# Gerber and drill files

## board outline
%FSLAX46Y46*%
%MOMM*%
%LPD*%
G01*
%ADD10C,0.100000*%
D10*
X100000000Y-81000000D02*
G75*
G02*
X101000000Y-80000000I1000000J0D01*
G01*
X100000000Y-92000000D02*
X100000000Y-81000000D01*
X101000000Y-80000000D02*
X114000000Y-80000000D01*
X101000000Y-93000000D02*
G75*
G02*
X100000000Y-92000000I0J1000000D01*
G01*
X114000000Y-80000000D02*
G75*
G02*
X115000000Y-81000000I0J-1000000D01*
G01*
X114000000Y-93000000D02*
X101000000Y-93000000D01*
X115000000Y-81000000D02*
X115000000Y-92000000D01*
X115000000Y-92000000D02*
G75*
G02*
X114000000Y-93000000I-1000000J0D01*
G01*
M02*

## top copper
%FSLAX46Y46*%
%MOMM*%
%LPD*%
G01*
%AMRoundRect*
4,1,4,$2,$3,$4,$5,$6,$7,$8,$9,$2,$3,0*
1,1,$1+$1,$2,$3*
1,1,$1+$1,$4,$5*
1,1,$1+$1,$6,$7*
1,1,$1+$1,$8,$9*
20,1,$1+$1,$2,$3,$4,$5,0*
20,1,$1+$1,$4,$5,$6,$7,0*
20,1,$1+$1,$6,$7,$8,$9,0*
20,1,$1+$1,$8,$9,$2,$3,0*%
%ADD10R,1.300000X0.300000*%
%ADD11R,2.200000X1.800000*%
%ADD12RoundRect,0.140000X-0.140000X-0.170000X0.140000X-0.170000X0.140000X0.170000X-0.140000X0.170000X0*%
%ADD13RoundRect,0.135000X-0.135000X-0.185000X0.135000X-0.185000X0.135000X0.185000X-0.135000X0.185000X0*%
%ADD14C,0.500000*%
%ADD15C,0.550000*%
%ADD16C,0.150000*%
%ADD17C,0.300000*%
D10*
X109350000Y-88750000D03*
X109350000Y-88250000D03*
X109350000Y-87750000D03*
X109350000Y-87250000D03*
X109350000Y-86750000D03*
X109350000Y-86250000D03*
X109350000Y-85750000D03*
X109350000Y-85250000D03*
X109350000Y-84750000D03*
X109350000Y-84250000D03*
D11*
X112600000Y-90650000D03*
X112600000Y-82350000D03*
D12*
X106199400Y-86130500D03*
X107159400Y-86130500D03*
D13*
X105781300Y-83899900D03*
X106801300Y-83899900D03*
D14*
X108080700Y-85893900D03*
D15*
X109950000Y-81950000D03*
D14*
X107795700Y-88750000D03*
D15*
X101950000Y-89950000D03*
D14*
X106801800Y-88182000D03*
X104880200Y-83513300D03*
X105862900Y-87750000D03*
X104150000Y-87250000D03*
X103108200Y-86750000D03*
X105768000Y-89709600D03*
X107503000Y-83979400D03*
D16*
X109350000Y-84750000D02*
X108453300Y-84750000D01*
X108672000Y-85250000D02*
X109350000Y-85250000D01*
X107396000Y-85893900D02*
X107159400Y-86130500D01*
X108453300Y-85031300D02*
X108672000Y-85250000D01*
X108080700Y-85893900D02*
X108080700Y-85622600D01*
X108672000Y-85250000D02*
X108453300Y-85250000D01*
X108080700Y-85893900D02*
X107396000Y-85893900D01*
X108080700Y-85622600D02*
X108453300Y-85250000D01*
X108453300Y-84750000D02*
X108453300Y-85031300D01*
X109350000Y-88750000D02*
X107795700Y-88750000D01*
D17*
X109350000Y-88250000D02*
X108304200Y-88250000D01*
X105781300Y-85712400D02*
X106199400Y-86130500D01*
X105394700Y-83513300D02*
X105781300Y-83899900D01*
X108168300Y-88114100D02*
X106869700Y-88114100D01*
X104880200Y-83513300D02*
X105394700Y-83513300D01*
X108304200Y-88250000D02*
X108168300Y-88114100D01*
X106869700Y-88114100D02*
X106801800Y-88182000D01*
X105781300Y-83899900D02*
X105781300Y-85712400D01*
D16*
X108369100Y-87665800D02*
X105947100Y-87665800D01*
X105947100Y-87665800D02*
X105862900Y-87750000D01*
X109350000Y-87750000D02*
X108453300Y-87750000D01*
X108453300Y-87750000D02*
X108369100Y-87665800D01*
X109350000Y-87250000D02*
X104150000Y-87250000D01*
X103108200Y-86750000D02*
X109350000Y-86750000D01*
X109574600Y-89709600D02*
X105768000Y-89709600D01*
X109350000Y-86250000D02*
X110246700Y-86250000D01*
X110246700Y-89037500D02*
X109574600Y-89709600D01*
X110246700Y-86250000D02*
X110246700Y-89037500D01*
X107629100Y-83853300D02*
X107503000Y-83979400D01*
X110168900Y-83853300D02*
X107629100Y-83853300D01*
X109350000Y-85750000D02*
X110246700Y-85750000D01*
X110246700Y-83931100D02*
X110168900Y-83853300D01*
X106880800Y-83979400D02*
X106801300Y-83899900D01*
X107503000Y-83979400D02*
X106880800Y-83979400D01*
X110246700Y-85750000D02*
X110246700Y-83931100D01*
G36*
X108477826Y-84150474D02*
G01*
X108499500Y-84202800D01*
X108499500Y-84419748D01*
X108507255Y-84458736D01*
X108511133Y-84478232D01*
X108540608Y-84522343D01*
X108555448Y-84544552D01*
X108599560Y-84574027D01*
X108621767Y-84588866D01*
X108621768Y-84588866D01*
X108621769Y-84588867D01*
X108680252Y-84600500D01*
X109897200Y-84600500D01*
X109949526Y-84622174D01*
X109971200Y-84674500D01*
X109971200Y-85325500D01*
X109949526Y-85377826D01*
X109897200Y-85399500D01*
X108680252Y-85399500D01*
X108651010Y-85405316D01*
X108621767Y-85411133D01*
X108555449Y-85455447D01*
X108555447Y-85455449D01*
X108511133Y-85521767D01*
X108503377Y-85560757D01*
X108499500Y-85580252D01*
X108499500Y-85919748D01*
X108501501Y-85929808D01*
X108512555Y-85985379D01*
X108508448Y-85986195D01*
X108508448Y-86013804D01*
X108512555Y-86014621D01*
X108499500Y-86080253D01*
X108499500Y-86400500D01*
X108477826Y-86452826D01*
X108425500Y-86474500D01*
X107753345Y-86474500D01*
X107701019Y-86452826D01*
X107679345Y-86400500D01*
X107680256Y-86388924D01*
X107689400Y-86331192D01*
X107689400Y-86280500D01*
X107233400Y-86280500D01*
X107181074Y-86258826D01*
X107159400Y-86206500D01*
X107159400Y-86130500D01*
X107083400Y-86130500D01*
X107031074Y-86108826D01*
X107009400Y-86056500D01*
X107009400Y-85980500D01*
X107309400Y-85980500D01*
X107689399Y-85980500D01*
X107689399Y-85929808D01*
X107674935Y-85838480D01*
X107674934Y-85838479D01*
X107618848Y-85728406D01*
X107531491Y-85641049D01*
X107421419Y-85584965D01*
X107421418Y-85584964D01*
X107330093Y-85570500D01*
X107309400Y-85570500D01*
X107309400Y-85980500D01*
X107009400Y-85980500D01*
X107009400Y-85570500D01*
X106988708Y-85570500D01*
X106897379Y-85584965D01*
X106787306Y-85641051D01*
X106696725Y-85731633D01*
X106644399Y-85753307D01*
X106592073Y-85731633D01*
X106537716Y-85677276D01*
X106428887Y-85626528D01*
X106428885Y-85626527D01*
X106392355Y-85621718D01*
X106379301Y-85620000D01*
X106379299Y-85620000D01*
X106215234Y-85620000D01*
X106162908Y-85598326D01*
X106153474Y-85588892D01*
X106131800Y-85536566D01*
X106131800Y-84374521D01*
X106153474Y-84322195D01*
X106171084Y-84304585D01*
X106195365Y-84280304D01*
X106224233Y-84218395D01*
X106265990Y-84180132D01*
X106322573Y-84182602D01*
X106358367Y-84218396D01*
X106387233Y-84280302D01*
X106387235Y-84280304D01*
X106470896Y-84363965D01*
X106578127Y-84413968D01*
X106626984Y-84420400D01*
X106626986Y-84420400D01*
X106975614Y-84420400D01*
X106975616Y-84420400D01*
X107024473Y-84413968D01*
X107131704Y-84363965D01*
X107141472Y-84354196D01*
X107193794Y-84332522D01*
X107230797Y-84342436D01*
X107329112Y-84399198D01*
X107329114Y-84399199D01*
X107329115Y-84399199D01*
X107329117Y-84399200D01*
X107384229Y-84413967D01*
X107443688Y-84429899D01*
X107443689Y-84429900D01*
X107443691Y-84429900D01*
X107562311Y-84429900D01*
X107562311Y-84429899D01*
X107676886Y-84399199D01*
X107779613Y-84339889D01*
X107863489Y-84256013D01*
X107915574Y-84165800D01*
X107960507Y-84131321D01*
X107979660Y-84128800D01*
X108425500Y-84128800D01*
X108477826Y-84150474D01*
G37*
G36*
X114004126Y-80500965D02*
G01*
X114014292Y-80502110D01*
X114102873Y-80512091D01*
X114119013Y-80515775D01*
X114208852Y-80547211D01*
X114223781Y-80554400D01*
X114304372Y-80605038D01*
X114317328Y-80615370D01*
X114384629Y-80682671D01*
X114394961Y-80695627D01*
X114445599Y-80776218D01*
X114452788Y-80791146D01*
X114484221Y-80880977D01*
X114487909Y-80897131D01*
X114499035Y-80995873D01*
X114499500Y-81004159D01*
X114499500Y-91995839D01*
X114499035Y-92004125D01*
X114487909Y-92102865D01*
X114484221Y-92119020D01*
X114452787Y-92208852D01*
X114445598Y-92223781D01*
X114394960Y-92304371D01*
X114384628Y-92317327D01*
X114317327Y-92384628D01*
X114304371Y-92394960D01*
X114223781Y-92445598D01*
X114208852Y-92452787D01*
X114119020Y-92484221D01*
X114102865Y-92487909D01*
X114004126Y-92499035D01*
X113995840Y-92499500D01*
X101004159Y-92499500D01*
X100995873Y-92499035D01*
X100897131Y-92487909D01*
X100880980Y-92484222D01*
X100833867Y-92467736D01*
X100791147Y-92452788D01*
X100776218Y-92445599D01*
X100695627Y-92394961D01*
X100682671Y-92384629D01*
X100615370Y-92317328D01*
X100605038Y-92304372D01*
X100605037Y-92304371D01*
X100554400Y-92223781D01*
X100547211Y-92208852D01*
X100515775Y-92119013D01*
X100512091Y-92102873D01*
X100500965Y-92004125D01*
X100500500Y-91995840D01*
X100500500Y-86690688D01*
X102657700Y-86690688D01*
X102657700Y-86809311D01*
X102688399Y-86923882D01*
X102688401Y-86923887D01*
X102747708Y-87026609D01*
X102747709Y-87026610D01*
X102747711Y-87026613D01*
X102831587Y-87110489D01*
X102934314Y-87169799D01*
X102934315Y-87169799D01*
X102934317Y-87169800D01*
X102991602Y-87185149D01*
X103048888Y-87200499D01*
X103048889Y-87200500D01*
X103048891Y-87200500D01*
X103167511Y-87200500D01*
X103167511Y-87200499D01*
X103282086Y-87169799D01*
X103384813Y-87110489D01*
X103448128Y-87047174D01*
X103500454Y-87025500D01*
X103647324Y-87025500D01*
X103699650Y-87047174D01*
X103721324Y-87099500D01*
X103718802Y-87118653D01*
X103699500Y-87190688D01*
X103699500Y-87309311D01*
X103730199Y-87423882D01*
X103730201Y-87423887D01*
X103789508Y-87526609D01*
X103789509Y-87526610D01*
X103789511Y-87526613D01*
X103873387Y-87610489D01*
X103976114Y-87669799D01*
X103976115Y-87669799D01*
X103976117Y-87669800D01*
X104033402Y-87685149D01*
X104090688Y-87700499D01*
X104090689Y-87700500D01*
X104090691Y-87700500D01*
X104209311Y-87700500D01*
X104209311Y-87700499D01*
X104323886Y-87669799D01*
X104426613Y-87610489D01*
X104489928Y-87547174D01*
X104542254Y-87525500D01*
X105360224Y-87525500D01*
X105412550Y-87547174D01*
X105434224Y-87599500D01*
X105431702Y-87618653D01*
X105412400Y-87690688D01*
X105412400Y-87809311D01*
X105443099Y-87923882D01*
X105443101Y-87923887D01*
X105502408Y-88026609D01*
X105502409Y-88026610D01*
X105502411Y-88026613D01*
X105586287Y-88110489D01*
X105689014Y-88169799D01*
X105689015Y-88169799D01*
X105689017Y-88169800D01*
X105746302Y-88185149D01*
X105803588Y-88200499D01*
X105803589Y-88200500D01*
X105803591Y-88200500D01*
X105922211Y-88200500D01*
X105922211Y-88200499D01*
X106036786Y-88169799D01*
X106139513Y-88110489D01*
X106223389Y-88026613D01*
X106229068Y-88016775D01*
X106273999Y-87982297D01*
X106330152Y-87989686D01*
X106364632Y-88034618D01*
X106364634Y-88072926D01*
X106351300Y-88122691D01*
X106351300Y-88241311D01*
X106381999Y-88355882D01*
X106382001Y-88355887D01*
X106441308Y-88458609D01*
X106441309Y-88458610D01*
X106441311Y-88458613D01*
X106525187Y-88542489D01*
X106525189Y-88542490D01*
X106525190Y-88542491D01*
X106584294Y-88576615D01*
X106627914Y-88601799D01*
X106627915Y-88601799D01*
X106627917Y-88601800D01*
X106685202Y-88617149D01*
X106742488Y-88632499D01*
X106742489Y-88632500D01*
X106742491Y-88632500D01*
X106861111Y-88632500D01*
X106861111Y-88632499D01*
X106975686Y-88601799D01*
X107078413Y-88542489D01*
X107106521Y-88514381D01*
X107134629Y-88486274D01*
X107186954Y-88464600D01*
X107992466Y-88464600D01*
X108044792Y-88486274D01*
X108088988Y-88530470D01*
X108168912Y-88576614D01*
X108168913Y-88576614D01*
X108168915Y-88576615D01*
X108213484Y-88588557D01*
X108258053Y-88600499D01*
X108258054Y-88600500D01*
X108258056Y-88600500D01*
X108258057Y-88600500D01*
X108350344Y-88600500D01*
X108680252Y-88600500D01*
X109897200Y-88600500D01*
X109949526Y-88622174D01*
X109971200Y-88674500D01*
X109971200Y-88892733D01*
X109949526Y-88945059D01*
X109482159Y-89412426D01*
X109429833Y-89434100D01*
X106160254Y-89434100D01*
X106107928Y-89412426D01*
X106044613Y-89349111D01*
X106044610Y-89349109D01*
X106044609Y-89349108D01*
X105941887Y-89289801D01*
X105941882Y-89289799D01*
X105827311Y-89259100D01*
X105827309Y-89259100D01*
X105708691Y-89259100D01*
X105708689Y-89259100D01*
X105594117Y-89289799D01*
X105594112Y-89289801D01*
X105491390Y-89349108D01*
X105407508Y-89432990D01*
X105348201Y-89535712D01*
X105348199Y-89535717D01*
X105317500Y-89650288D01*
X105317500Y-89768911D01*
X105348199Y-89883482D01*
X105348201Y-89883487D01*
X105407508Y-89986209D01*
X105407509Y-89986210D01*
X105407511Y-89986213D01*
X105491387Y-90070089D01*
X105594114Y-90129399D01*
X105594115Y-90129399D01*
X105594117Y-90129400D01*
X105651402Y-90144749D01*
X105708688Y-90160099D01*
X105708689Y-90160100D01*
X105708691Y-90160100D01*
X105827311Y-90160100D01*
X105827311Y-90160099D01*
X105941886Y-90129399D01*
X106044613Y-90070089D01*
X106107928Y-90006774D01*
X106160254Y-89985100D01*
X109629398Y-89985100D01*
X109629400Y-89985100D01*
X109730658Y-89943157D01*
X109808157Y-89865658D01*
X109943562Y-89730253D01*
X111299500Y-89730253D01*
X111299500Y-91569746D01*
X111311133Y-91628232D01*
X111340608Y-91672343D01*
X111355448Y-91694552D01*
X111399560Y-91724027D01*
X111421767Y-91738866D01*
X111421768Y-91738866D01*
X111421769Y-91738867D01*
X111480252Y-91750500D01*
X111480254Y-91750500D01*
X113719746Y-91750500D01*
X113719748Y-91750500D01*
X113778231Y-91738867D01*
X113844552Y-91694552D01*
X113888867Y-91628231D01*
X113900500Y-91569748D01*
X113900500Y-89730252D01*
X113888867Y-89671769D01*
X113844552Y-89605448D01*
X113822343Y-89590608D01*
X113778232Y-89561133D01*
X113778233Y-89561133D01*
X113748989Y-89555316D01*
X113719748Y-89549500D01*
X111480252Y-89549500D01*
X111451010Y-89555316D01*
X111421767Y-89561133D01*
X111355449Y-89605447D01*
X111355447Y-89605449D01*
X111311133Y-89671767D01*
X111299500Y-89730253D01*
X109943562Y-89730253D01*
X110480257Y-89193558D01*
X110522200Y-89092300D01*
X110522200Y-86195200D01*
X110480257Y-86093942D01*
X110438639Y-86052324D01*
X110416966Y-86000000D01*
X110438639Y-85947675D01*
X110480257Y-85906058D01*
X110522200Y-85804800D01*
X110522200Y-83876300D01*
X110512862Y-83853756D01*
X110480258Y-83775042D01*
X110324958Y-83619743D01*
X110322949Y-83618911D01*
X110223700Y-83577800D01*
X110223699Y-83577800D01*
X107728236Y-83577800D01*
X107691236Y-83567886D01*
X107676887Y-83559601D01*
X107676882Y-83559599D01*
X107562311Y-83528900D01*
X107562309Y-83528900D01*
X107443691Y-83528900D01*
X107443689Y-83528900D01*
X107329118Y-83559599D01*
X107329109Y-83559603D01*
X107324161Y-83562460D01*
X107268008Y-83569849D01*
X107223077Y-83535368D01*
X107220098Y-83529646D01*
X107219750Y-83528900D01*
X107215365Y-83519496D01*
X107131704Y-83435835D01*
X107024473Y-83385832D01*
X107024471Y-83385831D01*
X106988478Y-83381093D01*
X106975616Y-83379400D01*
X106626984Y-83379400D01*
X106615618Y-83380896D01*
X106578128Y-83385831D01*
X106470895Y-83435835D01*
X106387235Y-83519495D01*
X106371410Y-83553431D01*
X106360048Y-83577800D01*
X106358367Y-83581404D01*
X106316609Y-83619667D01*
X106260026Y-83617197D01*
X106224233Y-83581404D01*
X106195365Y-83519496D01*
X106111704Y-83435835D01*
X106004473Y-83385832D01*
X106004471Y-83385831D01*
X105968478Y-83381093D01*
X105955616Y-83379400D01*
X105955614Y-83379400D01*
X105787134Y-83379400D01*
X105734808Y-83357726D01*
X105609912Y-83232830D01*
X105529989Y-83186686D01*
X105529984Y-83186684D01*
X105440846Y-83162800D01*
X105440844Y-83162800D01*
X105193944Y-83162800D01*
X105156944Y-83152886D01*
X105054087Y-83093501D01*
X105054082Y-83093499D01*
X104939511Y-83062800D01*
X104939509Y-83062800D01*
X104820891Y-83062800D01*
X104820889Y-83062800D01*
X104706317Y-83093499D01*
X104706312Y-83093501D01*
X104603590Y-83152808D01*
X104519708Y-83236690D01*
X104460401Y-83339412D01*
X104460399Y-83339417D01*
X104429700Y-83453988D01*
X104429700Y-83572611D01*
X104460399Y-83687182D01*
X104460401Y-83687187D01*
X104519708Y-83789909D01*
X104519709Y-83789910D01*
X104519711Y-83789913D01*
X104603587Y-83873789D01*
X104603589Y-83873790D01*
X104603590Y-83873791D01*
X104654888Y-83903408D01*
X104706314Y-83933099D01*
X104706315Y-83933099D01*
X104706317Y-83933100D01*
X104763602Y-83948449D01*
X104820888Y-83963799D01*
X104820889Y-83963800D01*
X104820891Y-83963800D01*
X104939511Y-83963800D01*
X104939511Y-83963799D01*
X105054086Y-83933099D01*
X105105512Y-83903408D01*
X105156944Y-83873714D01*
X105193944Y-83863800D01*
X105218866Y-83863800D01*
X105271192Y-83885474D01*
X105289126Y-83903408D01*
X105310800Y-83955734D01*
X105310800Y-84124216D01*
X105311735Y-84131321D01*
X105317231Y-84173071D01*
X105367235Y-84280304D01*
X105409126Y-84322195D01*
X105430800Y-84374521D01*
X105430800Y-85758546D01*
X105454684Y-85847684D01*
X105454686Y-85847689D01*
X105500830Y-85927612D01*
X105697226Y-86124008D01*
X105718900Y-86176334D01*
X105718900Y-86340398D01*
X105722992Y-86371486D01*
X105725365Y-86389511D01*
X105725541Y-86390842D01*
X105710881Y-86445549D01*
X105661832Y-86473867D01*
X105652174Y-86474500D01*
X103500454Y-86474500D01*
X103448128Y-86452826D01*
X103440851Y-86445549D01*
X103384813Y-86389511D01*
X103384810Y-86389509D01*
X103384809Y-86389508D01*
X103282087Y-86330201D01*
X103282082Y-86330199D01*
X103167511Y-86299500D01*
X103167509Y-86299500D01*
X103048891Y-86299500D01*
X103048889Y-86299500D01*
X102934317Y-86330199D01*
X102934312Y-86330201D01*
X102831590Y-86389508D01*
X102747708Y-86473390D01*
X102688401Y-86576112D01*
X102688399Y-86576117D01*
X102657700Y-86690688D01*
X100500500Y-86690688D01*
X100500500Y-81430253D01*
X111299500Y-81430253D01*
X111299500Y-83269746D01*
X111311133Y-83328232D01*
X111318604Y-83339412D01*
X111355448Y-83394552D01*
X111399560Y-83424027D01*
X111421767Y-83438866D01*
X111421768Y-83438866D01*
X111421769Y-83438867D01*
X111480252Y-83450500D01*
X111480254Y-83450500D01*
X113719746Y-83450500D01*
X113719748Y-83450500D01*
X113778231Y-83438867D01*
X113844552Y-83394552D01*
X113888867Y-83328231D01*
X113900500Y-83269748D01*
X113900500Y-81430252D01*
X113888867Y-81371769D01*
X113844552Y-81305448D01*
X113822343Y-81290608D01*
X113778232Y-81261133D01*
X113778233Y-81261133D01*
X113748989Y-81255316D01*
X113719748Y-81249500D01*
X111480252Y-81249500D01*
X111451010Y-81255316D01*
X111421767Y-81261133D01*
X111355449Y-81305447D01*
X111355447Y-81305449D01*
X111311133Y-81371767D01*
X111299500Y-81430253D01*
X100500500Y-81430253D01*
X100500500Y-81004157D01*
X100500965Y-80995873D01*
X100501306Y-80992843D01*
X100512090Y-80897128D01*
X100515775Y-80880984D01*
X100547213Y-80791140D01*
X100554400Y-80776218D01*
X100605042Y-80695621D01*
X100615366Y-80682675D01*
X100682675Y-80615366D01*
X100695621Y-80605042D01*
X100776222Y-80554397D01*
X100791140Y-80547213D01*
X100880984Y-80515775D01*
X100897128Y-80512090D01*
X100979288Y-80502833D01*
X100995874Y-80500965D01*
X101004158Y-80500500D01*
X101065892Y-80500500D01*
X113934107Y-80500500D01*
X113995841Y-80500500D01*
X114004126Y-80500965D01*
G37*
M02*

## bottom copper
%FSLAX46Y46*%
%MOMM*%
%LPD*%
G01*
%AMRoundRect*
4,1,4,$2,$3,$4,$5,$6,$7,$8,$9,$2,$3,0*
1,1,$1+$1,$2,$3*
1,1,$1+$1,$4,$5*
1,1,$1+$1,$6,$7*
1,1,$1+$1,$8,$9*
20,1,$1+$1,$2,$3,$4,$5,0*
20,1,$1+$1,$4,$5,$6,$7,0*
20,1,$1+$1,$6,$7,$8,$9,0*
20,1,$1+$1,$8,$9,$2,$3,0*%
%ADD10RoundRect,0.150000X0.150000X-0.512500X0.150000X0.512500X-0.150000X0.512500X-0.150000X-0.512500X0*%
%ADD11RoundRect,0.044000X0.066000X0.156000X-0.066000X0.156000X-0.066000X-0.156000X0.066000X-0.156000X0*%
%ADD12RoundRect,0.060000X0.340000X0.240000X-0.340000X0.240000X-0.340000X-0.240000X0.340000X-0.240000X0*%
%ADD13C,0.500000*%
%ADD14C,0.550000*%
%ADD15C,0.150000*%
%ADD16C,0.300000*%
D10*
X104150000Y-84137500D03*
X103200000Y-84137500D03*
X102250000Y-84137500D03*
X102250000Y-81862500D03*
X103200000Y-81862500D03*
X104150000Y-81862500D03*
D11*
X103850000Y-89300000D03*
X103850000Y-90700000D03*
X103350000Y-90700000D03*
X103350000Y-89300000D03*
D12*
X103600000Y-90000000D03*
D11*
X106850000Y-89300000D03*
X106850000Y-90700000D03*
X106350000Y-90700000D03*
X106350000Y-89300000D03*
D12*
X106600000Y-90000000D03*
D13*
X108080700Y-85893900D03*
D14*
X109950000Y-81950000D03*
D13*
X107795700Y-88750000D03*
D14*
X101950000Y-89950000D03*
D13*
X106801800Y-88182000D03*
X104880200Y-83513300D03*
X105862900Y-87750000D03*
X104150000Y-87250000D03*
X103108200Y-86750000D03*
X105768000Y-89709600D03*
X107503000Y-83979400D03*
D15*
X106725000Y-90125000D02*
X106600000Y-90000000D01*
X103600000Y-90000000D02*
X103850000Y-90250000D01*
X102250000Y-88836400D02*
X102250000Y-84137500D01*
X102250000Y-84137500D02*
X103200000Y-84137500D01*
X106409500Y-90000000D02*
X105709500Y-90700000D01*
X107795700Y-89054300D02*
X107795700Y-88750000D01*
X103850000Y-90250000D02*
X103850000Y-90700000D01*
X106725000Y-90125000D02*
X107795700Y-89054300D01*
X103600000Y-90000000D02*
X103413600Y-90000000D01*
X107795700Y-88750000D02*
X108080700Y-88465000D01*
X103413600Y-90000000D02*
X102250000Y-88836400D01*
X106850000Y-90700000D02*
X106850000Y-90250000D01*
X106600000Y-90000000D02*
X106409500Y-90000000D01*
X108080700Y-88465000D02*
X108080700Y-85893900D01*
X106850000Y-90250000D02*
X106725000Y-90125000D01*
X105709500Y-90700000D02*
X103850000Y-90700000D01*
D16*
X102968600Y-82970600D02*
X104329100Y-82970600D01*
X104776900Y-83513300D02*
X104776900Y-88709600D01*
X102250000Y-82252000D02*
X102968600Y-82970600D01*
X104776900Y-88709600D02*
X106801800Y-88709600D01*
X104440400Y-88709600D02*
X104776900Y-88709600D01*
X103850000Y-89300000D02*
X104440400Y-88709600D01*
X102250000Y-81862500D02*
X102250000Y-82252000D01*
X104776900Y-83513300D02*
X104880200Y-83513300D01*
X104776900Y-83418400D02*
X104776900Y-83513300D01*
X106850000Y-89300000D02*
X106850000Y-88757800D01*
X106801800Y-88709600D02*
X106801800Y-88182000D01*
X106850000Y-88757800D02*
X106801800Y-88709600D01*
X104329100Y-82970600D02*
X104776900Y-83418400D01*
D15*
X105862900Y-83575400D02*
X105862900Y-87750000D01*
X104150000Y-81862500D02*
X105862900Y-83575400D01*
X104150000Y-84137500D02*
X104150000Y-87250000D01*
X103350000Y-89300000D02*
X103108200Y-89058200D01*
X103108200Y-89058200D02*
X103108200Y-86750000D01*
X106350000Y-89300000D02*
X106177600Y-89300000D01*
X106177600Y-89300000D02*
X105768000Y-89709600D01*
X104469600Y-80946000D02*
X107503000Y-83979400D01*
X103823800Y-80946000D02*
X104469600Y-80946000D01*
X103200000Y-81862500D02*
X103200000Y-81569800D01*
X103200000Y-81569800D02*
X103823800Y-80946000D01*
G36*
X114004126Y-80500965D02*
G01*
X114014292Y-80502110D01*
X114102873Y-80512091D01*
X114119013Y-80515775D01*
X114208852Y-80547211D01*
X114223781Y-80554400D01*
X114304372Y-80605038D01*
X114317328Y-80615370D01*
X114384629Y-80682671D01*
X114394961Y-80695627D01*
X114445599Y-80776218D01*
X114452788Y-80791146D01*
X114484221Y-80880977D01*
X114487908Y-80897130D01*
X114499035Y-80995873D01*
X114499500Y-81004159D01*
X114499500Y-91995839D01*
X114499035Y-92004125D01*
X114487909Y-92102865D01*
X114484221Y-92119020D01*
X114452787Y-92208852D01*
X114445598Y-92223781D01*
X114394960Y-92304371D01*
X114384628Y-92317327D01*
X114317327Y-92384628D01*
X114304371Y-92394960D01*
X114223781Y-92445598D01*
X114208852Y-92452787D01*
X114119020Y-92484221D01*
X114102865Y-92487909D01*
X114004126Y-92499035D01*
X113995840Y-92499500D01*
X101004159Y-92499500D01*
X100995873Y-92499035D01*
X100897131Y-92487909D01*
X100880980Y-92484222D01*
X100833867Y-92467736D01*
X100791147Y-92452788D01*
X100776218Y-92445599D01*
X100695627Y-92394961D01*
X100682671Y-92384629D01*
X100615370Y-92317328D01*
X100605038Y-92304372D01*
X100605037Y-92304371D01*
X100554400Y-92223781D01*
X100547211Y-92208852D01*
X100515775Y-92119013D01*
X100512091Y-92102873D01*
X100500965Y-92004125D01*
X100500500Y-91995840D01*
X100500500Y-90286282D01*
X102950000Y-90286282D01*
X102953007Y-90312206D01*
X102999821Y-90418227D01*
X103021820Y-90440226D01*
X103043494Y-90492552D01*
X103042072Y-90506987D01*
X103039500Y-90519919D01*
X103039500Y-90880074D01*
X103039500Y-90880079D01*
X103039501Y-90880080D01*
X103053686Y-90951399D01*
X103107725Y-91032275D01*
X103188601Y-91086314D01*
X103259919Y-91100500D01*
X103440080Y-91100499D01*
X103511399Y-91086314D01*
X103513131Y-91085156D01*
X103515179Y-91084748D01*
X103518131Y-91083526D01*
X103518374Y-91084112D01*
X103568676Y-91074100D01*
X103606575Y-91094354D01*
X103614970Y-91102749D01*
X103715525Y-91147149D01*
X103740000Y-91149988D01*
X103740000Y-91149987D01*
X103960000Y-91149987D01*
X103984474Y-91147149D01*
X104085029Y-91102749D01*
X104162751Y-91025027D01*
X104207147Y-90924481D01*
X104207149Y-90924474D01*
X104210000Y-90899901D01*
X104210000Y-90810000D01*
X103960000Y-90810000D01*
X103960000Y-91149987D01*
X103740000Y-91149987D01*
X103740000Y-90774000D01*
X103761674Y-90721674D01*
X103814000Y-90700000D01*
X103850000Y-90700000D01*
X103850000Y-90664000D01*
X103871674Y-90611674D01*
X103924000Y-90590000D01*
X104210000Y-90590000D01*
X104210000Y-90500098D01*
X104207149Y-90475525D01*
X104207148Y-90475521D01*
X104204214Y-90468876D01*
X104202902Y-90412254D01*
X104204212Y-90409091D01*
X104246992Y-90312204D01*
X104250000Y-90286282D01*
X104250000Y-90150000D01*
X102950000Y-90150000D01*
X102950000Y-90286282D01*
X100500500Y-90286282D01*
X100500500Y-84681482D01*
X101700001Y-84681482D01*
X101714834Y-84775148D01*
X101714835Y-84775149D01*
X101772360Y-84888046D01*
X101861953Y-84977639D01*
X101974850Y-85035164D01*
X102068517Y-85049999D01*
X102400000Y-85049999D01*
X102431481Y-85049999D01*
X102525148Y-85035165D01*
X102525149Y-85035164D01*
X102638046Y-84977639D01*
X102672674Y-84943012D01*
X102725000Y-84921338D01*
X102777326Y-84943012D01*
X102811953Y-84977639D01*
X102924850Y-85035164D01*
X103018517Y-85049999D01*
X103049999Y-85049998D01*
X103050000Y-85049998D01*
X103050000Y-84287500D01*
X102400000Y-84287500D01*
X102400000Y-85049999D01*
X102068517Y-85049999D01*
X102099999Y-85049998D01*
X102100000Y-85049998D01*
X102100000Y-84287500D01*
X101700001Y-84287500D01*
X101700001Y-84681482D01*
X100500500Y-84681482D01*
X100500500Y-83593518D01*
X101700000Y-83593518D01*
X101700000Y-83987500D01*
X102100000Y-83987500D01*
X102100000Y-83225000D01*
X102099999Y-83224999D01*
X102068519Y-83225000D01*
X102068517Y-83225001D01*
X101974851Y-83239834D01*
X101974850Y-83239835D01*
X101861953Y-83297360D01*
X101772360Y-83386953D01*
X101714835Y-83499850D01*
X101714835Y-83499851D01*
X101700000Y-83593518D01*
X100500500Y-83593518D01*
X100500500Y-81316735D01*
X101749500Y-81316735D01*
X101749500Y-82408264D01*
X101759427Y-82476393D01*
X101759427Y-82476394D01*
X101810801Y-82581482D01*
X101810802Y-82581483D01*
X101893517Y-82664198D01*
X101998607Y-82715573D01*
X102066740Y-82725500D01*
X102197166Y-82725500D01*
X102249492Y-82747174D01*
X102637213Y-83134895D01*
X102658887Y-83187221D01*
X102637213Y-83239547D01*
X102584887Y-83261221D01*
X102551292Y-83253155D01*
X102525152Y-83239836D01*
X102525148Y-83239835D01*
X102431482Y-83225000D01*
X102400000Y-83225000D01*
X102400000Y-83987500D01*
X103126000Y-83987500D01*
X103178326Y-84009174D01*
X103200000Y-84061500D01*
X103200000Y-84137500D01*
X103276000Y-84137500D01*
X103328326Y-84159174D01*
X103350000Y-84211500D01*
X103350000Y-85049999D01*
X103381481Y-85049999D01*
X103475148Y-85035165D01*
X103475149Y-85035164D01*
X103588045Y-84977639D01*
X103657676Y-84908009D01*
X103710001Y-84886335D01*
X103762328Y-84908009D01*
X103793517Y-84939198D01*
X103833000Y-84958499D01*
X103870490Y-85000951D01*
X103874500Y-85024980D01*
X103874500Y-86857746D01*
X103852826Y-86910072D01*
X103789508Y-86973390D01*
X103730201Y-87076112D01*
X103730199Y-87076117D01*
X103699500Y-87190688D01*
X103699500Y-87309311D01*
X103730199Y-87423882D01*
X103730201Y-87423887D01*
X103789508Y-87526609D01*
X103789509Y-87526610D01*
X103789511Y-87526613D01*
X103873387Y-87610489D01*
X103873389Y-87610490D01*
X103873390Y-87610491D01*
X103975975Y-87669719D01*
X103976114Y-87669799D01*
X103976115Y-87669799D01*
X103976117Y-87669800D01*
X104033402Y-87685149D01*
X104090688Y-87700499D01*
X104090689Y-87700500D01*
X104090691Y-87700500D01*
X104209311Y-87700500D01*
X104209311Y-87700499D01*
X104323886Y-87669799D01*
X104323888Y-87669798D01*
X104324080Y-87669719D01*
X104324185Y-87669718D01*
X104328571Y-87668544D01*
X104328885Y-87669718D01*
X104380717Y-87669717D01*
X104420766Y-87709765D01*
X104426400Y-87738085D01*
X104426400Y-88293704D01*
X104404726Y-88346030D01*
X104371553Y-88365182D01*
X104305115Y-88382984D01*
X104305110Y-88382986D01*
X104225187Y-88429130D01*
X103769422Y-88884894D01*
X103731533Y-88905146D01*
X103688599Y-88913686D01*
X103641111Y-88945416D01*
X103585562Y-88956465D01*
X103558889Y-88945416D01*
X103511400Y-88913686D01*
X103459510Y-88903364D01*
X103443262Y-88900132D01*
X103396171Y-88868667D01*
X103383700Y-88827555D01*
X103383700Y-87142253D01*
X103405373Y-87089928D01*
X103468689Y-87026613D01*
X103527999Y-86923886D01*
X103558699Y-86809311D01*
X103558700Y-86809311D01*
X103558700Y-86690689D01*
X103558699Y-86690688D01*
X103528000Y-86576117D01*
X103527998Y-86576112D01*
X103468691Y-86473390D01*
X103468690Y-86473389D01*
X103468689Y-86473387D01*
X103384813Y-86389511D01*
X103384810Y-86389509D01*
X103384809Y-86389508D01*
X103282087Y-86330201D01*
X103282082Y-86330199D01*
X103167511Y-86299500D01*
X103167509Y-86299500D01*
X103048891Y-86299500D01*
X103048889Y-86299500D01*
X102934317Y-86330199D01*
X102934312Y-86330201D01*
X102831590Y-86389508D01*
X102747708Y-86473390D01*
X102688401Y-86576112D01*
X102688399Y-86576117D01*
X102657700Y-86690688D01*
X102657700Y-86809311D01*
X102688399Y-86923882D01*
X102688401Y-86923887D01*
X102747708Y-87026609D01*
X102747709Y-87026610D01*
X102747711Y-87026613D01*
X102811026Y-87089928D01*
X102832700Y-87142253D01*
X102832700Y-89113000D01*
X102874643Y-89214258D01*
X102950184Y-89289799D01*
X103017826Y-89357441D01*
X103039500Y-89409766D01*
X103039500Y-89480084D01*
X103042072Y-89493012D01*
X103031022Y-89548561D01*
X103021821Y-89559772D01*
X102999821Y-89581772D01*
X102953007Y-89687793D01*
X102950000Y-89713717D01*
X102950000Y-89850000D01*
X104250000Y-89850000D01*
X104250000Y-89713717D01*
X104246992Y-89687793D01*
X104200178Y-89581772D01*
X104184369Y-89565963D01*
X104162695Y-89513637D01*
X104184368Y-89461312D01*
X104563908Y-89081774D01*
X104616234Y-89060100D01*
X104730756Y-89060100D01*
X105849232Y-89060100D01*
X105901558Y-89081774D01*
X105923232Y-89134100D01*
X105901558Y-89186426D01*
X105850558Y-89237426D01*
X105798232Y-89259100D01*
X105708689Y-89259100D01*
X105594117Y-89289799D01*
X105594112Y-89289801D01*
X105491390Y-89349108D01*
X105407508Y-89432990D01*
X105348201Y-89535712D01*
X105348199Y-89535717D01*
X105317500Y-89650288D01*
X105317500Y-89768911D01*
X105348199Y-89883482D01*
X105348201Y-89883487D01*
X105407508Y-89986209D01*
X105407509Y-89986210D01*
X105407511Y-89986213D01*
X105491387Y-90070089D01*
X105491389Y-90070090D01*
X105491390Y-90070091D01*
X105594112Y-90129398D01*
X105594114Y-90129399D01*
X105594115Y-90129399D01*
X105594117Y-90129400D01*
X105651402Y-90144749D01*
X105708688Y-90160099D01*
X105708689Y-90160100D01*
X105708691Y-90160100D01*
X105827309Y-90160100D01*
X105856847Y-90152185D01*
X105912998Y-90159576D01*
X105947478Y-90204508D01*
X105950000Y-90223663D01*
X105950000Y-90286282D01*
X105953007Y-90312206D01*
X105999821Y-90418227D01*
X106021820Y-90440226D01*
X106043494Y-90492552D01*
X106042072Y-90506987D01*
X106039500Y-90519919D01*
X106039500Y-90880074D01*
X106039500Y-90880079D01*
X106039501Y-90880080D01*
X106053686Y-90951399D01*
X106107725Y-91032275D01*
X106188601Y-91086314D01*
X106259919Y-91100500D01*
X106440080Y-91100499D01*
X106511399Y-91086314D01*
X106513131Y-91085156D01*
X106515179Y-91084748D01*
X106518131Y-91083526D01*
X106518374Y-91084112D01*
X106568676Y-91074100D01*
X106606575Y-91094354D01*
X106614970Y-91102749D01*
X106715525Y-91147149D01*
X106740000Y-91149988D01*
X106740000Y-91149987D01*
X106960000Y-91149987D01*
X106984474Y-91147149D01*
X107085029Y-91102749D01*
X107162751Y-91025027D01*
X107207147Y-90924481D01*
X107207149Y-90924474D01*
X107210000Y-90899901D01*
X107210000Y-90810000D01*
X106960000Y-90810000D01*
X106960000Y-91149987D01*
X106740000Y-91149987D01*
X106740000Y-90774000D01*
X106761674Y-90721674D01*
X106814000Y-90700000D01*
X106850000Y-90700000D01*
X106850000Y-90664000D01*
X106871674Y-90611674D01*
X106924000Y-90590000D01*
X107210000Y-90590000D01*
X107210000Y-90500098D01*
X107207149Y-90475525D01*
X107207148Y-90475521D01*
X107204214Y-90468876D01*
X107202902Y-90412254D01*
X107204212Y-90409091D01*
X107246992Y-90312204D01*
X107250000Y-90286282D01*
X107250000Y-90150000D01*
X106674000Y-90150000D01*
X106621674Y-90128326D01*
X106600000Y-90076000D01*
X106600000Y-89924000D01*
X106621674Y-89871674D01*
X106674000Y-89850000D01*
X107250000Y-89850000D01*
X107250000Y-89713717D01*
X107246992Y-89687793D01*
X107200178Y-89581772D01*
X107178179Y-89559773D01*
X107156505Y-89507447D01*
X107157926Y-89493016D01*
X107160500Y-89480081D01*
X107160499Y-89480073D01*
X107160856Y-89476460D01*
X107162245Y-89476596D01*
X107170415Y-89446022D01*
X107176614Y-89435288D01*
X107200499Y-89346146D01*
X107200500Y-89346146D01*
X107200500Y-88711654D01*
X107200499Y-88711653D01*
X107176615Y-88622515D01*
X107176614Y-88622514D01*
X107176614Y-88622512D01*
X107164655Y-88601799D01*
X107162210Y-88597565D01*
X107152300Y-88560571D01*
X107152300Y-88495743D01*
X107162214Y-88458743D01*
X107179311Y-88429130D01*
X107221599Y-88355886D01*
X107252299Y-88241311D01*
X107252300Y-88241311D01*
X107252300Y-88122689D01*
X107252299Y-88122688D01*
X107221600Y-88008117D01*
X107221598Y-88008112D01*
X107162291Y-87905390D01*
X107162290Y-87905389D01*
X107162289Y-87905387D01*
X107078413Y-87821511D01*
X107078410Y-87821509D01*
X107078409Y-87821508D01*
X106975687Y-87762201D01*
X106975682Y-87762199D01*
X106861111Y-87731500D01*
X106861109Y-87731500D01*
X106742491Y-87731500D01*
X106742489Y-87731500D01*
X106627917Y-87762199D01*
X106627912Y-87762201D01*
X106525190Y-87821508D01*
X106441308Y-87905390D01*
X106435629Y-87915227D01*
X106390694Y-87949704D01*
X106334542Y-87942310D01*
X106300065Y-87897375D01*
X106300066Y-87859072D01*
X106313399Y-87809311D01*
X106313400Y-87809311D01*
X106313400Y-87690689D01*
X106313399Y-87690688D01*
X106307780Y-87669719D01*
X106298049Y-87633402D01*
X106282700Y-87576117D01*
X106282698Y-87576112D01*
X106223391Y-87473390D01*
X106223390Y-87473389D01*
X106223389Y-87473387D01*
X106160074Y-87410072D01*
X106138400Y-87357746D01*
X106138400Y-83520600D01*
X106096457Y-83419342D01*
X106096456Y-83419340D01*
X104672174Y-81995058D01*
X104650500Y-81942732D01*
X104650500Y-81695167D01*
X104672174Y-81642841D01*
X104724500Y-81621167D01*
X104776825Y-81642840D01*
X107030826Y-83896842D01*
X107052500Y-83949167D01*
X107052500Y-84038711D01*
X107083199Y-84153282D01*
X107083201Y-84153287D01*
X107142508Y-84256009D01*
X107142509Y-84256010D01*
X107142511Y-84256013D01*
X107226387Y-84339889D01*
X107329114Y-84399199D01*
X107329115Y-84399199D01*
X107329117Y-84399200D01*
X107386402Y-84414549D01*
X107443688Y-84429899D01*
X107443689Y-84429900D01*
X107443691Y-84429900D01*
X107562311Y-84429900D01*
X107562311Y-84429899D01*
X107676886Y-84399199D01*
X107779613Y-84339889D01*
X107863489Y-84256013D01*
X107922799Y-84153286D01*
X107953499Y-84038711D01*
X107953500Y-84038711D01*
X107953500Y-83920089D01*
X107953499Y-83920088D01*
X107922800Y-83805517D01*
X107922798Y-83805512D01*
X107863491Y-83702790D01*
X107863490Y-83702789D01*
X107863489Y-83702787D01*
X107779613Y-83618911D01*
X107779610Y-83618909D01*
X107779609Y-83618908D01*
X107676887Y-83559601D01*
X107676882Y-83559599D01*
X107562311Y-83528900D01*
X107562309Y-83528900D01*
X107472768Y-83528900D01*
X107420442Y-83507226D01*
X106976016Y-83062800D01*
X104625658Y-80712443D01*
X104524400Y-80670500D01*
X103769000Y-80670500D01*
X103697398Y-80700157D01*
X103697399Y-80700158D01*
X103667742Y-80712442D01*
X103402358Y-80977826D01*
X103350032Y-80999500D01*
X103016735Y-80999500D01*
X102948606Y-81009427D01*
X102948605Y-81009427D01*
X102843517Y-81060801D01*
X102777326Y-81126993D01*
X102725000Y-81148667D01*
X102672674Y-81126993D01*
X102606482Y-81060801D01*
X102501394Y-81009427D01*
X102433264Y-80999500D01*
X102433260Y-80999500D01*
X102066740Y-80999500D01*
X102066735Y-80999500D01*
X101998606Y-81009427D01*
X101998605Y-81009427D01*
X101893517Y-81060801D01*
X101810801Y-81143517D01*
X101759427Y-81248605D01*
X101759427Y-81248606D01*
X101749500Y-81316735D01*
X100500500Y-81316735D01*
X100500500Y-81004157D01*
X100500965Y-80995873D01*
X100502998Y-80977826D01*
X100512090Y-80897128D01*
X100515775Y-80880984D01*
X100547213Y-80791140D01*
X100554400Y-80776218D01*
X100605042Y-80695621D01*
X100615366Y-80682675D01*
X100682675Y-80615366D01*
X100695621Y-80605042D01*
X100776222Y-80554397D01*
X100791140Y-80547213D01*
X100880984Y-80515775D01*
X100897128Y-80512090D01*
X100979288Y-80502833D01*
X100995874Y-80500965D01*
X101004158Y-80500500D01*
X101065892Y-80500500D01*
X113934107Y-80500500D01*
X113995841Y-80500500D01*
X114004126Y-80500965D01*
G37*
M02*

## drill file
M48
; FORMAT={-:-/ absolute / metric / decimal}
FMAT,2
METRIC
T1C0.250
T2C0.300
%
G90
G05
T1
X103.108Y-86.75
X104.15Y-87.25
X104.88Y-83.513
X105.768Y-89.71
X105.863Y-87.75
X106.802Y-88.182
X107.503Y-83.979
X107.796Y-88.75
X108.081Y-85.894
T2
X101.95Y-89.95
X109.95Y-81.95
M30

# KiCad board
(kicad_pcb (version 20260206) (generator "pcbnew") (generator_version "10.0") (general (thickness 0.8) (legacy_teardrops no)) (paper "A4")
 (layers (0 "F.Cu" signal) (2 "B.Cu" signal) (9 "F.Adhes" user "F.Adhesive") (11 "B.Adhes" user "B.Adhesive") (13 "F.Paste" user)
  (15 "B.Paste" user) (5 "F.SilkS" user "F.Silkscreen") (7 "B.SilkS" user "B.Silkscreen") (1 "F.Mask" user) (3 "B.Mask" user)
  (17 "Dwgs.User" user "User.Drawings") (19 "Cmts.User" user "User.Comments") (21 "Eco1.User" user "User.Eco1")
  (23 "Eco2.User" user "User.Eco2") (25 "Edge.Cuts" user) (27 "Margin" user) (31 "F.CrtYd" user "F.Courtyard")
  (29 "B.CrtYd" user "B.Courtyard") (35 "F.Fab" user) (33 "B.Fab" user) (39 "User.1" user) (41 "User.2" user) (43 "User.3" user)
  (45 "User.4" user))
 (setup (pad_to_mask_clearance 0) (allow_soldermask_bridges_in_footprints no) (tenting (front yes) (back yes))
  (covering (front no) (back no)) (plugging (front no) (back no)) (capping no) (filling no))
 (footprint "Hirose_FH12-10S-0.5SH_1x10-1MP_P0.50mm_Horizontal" (layer "F.Cu") (at 111.2 86.5 90)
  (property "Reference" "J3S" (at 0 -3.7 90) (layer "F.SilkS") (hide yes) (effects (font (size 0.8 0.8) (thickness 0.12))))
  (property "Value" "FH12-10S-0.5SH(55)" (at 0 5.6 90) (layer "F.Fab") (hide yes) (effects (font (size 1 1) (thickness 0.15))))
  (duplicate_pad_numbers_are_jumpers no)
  (pad "1" smd rect (at -2.25 -1.85 90) (size 0.3 1.3) (layers "F.Cu" "F.Mask" "F.Paste") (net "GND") (zone_connect 2))
  (pad "2" smd rect (at -1.75 -1.85 90) (size 0.3 1.3) (layers "F.Cu" "F.Mask" "F.Paste") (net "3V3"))
  (pad "3" smd rect (at -1.25 -1.85 90) (size 0.3 1.3) (layers "F.Cu" "F.Mask" "F.Paste") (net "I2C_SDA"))
  (pad "4" smd rect (at -0.75 -1.85 90) (size 0.3 1.3) (layers "F.Cu" "F.Mask" "F.Paste") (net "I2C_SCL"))
  (pad "5" smd rect (at -0.25 -1.85 90) (size 0.3 1.3) (layers "F.Cu" "F.Mask" "F.Paste") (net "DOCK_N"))
  (pad "6" smd rect (at 0.25 -1.85 90) (size 0.3 1.3) (layers "F.Cu" "F.Mask" "F.Paste") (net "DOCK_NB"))
  (pad "7" smd rect (at 0.75 -1.85 90) (size 0.3 1.3) (layers "F.Cu" "F.Mask" "F.Paste") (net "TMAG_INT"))
  (pad "8" smd rect (at 1.25 -1.85 90) (size 0.3 1.3) (layers "F.Cu" "F.Mask" "F.Paste") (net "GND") (zone_connect 2))
  (pad "9" smd rect (at 1.75 -1.85 90) (size 0.3 1.3) (layers "F.Cu" "F.Mask" "F.Paste") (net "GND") (zone_connect 2))
  (pad "10" smd rect (at 2.25 -1.85 90) (size 0.3 1.3) (layers "F.Cu" "F.Mask" "F.Paste"))
  (pad "MP" smd rect (at -4.15 1.4 90) (size 1.8 2.2) (layers "F.Cu" "F.Mask" "F.Paste"))
  (pad "MP" smd rect (at 4.15 1.4 90) (size 1.8 2.2) (layers "F.Cu" "F.Mask" "F.Paste")))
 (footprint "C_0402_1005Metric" (layer "F.Cu") (at 106.6794 86.1305)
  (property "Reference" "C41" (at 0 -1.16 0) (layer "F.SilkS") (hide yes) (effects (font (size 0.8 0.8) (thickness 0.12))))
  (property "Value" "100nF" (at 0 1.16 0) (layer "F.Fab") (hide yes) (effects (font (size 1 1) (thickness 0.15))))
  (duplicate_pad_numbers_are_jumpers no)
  (pad "1" smd roundrect (at -0.48 0) (size 0.56 0.62) (layers "F.Cu" "F.Mask" "F.Paste") (roundrect_rratio 0.25) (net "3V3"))
  (pad "2" smd roundrect (at 0.48 0) (size 0.56 0.62) (layers "F.Cu" "F.Mask" "F.Paste") (roundrect_rratio 0.25) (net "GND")))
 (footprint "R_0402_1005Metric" (layer "F.Cu") (at 106.2913 83.8999)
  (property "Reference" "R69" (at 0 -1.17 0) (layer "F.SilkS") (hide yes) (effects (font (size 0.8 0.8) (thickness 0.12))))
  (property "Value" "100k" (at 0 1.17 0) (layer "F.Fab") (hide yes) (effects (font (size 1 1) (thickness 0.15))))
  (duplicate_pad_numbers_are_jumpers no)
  (pad "1" smd roundrect (at -0.51 0) (size 0.54 0.64) (layers "F.Cu" "F.Mask" "F.Paste") (roundrect_rratio 0.25) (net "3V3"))
  (pad "2" smd roundrect (at 0.51 0) (size 0.54 0.64) (layers "F.Cu" "F.Mask" "F.Paste") (roundrect_rratio 0.25) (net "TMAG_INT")))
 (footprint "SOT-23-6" (layer "B.Cu") (at 103.2 83 90)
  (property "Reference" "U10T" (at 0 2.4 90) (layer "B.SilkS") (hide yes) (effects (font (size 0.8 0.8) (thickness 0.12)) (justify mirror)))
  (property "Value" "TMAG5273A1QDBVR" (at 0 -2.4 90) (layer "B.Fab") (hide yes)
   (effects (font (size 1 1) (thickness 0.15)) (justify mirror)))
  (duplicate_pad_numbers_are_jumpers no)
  (pad "1" smd roundrect (at -1.1375 0.95 90) (size 1.325 0.6) (layers "B.Cu" "B.Mask" "B.Paste") (roundrect_rratio 0.25) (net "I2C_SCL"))
  (pad "2" smd roundrect (at -1.1375 0 90) (size 1.325 0.6) (layers "B.Cu" "B.Mask" "B.Paste") (roundrect_rratio 0.25) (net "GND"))
  (pad "3" smd roundrect (at -1.1375 -0.95 90) (size 1.325 0.6) (layers "B.Cu" "B.Mask" "B.Paste") (roundrect_rratio 0.25) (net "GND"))
  (pad "4" smd roundrect (at 1.1375 -0.95 90) (size 1.325 0.6) (layers "B.Cu" "B.Mask" "B.Paste") (roundrect_rratio 0.25) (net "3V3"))
  (pad "5" smd roundrect (at 1.1375 0 90) (size 1.325 0.6) (layers "B.Cu" "B.Mask" "B.Paste") (roundrect_rratio 0.25) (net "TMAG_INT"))
  (pad "6" smd roundrect (at 1.1375 0.95 90) (size 1.325 0.6) (layers "B.Cu" "B.Mask" "B.Paste") (roundrect_rratio 0.25) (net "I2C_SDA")))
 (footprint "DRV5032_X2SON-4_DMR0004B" (layer "B.Cu") (at 103.6 90 180)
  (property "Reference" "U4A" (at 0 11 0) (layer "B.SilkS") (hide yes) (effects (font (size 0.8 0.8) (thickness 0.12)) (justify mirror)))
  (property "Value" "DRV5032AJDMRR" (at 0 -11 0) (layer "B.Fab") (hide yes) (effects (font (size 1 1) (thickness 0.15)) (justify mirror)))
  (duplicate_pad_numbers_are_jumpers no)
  (pad "1" smd roundrect (at -0.25 0.7 180) (size 0.22 0.4) (layers "B.Cu" "B.Mask" "B.Paste") (roundrect_rratio 0.2) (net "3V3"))
  (pad "2" smd roundrect (at -0.25 -0.7 180) (size 0.22 0.4) (layers "B.Cu" "B.Mask" "B.Paste") (roundrect_rratio 0.2) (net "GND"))
  (pad "3" smd roundrect (at 0.25 -0.7 180) (size 0.22 0.4) (layers "B.Cu" "B.Mask" "B.Paste") (roundrect_rratio 0.2))
  (pad "4" smd roundrect (at 0.25 0.7 180) (size 0.22 0.4) (layers "B.Cu" "B.Mask" "B.Paste") (roundrect_rratio 0.2) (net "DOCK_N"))
  (pad "5" smd roundrect (at 0 0 180) (size 0.8 0.6) (layers "B.Cu" "B.Mask" "B.Paste") (roundrect_rratio 0.1) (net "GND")))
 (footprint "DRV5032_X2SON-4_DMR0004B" (layer "B.Cu") (at 106.6 90 180)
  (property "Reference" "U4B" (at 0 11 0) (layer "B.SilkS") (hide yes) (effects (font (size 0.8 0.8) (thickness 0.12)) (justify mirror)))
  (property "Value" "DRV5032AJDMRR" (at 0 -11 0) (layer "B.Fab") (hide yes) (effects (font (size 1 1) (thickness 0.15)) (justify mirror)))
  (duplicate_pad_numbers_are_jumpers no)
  (pad "1" smd roundrect (at -0.25 0.7 180) (size 0.22 0.4) (layers "B.Cu" "B.Mask" "B.Paste") (roundrect_rratio 0.2) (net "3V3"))
  (pad "2" smd roundrect (at -0.25 -0.7 180) (size 0.22 0.4) (layers "B.Cu" "B.Mask" "B.Paste") (roundrect_rratio 0.2) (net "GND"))
  (pad "3" smd roundrect (at 0.25 -0.7 180) (size 0.22 0.4) (layers "B.Cu" "B.Mask" "B.Paste") (roundrect_rratio 0.2))
  (pad "4" smd roundrect (at 0.25 0.7 180) (size 0.22 0.4) (layers "B.Cu" "B.Mask" "B.Paste") (roundrect_rratio 0.2) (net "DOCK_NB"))
  (pad "5" smd roundrect (at 0 0 180) (size 0.8 0.6) (layers "B.Cu" "B.Mask" "B.Paste") (roundrect_rratio 0.1) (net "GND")))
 (gr_arc (start 100 81) (mid 100.292893 80.292893) (end 101 80) (stroke (width 0.1) (type default)) (layer "Edge.Cuts"))
 (gr_line (start 100 92) (end 100 81) (stroke (width 0.1) (type default)) (layer "Edge.Cuts"))
 (gr_line (start 101 80) (end 114 80) (stroke (width 0.1) (type default)) (layer "Edge.Cuts"))
 (gr_arc (start 101 93) (mid 100.292893 92.707106) (end 100 92) (stroke (width 0.1) (type default)) (layer "Edge.Cuts"))
 (gr_arc (start 114 80) (mid 114.707106 80.292893) (end 115 81) (stroke (width 0.1) (type default)) (layer "Edge.Cuts"))
 (gr_line (start 114 93) (end 101 93) (stroke (width 0.1) (type default)) (layer "Edge.Cuts"))
 (gr_line (start 115 81) (end 115 92) (stroke (width 0.1) (type default)) (layer "Edge.Cuts"))
 (gr_arc (start 115 92) (mid 114.707106 92.707106) (end 114 93) (stroke (width 0.1) (type default)) (layer "Edge.Cuts"))
 (segment (start 109.35 84.75) (end 108.4533 84.75) (width 0.15) (layer "F.Cu") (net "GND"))
 (segment (start 108.672 85.25) (end 109.35 85.25) (width 0.15) (layer "F.Cu") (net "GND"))
 (segment (start 107.396 85.8939) (end 107.1594 86.1305) (width 0.15) (layer "F.Cu") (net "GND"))
 (segment (start 108.4533 85.0313) (end 108.672 85.25) (width 0.15) (layer "F.Cu") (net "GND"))
 (segment (start 108.0807 85.8939) (end 108.0807 85.6226) (width 0.15) (layer "F.Cu") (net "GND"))
 (segment (start 108.672 85.25) (end 108.4533 85.25) (width 0.15) (layer "F.Cu") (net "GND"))
 (segment (start 108.0807 85.8939) (end 107.396 85.8939) (width 0.15) (layer "F.Cu") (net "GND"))
 (segment (start 108.0807 85.6226) (end 108.4533 85.25) (width 0.15) (layer "F.Cu") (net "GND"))
 (segment (start 108.4533 84.75) (end 108.4533 85.0313) (width 0.15) (layer "F.Cu") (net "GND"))
 (segment (start 109.35 88.75) (end 107.7957 88.75) (width 0.15) (layer "F.Cu") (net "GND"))
 (via (at 108.0807 85.8939) (size 0.5) (drill 0.25) (layers "F.Cu" "B.Cu") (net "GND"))
 (via (at 109.95 81.95) (size 0.55) (drill 0.3) (layers "F.Cu" "B.Cu") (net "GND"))
 (via (at 107.7957 88.75) (size 0.5) (drill 0.25) (layers "F.Cu" "B.Cu") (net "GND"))
 (via (at 101.95 89.95) (size 0.55) (drill 0.3) (layers "F.Cu" "B.Cu") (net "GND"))
 (segment (start 106.725 90.125) (end 106.6 90) (width 0.15) (layer "B.Cu") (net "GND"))
 (segment (start 103.6 90) (end 103.85 90.25) (width 0.15) (layer "B.Cu") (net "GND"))
 (segment (start 102.25 88.8364) (end 102.25 84.1375) (width 0.15) (layer "B.Cu") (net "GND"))
 (segment (start 102.25 84.1375) (end 103.2 84.1375) (width 0.15) (layer "B.Cu") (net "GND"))
 (segment (start 106.4095 90) (end 105.7095 90.7) (width 0.15) (layer "B.Cu") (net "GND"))
 (segment (start 107.7957 89.0543) (end 107.7957 88.75) (width 0.15) (layer "B.Cu") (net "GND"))
 (segment (start 103.85 90.25) (end 103.85 90.7) (width 0.15) (layer "B.Cu") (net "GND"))
 (segment (start 106.725 90.125) (end 107.7957 89.0543) (width 0.15) (layer "B.Cu") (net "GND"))
 (segment (start 103.6 90) (end 103.4136 90) (width 0.15) (layer "B.Cu") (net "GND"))
 (segment (start 107.7957 88.75) (end 108.0807 88.465) (width 0.15) (layer "B.Cu") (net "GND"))
 (segment (start 103.4136 90) (end 102.25 88.8364) (width 0.15) (layer "B.Cu") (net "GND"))
 (segment (start 106.85 90.7) (end 106.85 90.25) (width 0.15) (layer "B.Cu") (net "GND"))
 (segment (start 106.6 90) (end 106.4095 90) (width 0.15) (layer "B.Cu") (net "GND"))
 (segment (start 108.0807 88.465) (end 108.0807 85.8939) (width 0.15) (layer "B.Cu") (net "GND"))
 (segment (start 106.85 90.25) (end 106.725 90.125) (width 0.15) (layer "B.Cu") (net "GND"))
 (segment (start 105.7095 90.7) (end 103.85 90.7) (width 0.15) (layer "B.Cu") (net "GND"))
 (segment (start 109.35 88.25) (end 108.3042 88.25) (width 0.3) (layer "F.Cu") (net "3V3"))
 (segment (start 105.7813 85.7124) (end 106.1994 86.1305) (width 0.3) (layer "F.Cu") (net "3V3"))
 (segment (start 105.3947 83.5133) (end 105.7813 83.8999) (width 0.3) (layer "F.Cu") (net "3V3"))
 (segment (start 108.1683 88.1141) (end 106.8697 88.1141) (width 0.3) (layer "F.Cu") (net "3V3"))
 (segment (start 104.8802 83.5133) (end 105.3947 83.5133) (width 0.3) (layer "F.Cu") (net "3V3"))
 (segment (start 108.3042 88.25) (end 108.1683 88.1141) (width 0.3) (layer "F.Cu") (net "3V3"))
 (segment (start 106.8697 88.1141) (end 106.8018 88.182) (width 0.3) (layer "F.Cu") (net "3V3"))
 (segment (start 105.7813 83.8999) (end 105.7813 85.7124) (width 0.3) (layer "F.Cu") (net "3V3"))
 (via (at 106.8018 88.182) (size 0.5) (drill 0.25) (layers "F.Cu" "B.Cu") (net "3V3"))
 (via (at 104.8802 83.5133) (size 0.5) (drill 0.25) (layers "F.Cu" "B.Cu") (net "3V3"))
 (segment (start 102.9686 82.9706) (end 104.3291 82.9706) (width 0.3) (layer "B.Cu") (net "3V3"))
 (segment (start 104.7769 83.5133) (end 104.7769 88.7096) (width 0.3) (layer "B.Cu") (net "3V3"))
 (segment (start 102.25 82.252) (end 102.9686 82.9706) (width 0.3) (layer "B.Cu") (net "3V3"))
 (segment (start 104.7769 88.7096) (end 106.8018 88.7096) (width 0.3) (layer "B.Cu") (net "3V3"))
 (segment (start 104.4404 88.7096) (end 104.7769 88.7096) (width 0.3) (layer "B.Cu") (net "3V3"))
 (segment (start 103.85 89.3) (end 104.4404 88.7096) (width 0.3) (layer "B.Cu") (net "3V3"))
 (segment (start 102.25 81.8625) (end 102.25 82.252) (width 0.3) (layer "B.Cu") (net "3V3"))
 (segment (start 104.7769 83.5133) (end 104.8802 83.5133) (width 0.3) (layer "B.Cu") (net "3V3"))
 (segment (start 104.7769 83.4184) (end 104.7769 83.5133) (width 0.3) (layer "B.Cu") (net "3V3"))
 (segment (start 106.85 89.3) (end 106.85 88.7578) (width 0.3) (layer "B.Cu") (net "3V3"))
 (segment (start 106.8018 88.7096) (end 106.8018 88.182) (width 0.3) (layer "B.Cu") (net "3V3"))
 (segment (start 106.85 88.7578) (end 106.8018 88.7096) (width 0.3) (layer "B.Cu") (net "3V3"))
 (segment (start 104.3291 82.9706) (end 104.7769 83.4184) (width 0.3) (layer "B.Cu") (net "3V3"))
 (segment (start 108.3691 87.6658) (end 105.9471 87.6658) (width 0.15) (layer "F.Cu") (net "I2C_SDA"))
 (segment (start 105.9471 87.6658) (end 105.8629 87.75) (width 0.15) (layer "F.Cu") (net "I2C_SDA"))
 (segment (start 109.35 87.75) (end 108.4533 87.75) (width 0.15) (layer "F.Cu") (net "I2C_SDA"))
 (segment (start 108.4533 87.75) (end 108.3691 87.6658) (width 0.15) (layer "F.Cu") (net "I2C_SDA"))
 (via (at 105.8629 87.75) (size 0.5) (drill 0.25) (layers "F.Cu" "B.Cu") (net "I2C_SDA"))
 (segment (start 105.8629 83.5754) (end 105.8629 87.75) (width 0.15) (layer "B.Cu") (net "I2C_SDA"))
 (segment (start 104.15 81.8625) (end 105.8629 83.5754) (width 0.15) (layer "B.Cu") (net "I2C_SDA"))
 (segment (start 109.35 87.25) (end 104.15 87.25) (width 0.15) (layer "F.Cu") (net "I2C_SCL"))
 (via (at 104.15 87.25) (size 0.5) (drill 0.25) (layers "F.Cu" "B.Cu") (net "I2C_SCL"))
 (segment (start 104.15 84.1375) (end 104.15 87.25) (width 0.15) (layer "B.Cu") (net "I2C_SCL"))
 (segment (start 103.1082 86.75) (end 109.35 86.75) (width 0.15) (layer "F.Cu") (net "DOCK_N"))
 (via (at 103.1082 86.75) (size 0.5) (drill 0.25) (layers "F.Cu" "B.Cu") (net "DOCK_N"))
 (segment (start 103.35 89.3) (end 103.1082 89.0582) (width 0.15) (layer "B.Cu") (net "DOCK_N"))
 (segment (start 103.1082 89.0582) (end 103.1082 86.75) (width 0.15) (layer "B.Cu") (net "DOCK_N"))
 (segment (start 109.5746 89.7096) (end 105.768 89.7096) (width 0.15) (layer "F.Cu") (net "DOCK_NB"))
 (segment (start 109.35 86.25) (end 110.2467 86.25) (width 0.15) (layer "F.Cu") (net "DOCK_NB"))
 (segment (start 110.2467 89.0375) (end 109.5746 89.7096) (width 0.15) (layer "F.Cu") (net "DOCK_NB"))
 (segment (start 110.2467 86.25) (end 110.2467 89.0375) (width 0.15) (layer "F.Cu") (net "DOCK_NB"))
 (via (at 105.768 89.7096) (size 0.5) (drill 0.25) (layers "F.Cu" "B.Cu") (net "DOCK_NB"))
 (segment (start 106.35 89.3) (end 106.1776 89.3) (width 0.15) (layer "B.Cu") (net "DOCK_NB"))
 (segment (start 106.1776 89.3) (end 105.768 89.7096) (width 0.15) (layer "B.Cu") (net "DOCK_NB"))
 (segment (start 107.6291 83.8533) (end 107.503 83.9794) (width 0.15) (layer "F.Cu") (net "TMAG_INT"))
 (segment (start 110.1689 83.8533) (end 107.6291 83.8533) (width 0.15) (layer "F.Cu") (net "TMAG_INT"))
 (segment (start 109.35 85.75) (end 110.2467 85.75) (width 0.15) (layer "F.Cu") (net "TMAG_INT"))
 (segment (start 110.2467 83.9311) (end 110.1689 83.8533) (width 0.15) (layer "F.Cu") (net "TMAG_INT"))
 (segment (start 106.8808 83.9794) (end 106.8013 83.8999) (width 0.15) (layer "F.Cu") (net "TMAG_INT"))
 (segment (start 107.503 83.9794) (end 106.8808 83.9794) (width 0.15) (layer "F.Cu") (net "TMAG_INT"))
 (segment (start 110.2467 85.75) (end 110.2467 83.9311) (width 0.15) (layer "F.Cu") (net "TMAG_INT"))
 (via (at 107.503 83.9794) (size 0.5) (drill 0.25) (layers "F.Cu" "B.Cu") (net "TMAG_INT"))
 (segment (start 104.4696 80.946) (end 107.503 83.9794) (width 0.15) (layer "B.Cu") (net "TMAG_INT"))
 (segment (start 103.8238 80.946) (end 104.4696 80.946) (width 0.15) (layer "B.Cu") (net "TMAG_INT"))
 (segment (start 103.2 81.8625) (end 103.2 81.5698) (width 0.15) (layer "B.Cu") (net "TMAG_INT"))
 (segment (start 103.2 81.5698) (end 103.8238 80.946) (width 0.15) (layer "B.Cu") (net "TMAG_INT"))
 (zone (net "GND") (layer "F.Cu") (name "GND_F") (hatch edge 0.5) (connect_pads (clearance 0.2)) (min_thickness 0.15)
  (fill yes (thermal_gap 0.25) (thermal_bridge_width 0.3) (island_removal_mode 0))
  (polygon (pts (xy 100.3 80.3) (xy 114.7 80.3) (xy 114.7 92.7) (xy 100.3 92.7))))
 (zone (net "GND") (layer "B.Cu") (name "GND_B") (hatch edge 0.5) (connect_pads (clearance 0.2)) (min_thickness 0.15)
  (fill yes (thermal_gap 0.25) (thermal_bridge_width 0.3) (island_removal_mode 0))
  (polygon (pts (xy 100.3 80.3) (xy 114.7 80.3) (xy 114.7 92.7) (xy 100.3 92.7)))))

